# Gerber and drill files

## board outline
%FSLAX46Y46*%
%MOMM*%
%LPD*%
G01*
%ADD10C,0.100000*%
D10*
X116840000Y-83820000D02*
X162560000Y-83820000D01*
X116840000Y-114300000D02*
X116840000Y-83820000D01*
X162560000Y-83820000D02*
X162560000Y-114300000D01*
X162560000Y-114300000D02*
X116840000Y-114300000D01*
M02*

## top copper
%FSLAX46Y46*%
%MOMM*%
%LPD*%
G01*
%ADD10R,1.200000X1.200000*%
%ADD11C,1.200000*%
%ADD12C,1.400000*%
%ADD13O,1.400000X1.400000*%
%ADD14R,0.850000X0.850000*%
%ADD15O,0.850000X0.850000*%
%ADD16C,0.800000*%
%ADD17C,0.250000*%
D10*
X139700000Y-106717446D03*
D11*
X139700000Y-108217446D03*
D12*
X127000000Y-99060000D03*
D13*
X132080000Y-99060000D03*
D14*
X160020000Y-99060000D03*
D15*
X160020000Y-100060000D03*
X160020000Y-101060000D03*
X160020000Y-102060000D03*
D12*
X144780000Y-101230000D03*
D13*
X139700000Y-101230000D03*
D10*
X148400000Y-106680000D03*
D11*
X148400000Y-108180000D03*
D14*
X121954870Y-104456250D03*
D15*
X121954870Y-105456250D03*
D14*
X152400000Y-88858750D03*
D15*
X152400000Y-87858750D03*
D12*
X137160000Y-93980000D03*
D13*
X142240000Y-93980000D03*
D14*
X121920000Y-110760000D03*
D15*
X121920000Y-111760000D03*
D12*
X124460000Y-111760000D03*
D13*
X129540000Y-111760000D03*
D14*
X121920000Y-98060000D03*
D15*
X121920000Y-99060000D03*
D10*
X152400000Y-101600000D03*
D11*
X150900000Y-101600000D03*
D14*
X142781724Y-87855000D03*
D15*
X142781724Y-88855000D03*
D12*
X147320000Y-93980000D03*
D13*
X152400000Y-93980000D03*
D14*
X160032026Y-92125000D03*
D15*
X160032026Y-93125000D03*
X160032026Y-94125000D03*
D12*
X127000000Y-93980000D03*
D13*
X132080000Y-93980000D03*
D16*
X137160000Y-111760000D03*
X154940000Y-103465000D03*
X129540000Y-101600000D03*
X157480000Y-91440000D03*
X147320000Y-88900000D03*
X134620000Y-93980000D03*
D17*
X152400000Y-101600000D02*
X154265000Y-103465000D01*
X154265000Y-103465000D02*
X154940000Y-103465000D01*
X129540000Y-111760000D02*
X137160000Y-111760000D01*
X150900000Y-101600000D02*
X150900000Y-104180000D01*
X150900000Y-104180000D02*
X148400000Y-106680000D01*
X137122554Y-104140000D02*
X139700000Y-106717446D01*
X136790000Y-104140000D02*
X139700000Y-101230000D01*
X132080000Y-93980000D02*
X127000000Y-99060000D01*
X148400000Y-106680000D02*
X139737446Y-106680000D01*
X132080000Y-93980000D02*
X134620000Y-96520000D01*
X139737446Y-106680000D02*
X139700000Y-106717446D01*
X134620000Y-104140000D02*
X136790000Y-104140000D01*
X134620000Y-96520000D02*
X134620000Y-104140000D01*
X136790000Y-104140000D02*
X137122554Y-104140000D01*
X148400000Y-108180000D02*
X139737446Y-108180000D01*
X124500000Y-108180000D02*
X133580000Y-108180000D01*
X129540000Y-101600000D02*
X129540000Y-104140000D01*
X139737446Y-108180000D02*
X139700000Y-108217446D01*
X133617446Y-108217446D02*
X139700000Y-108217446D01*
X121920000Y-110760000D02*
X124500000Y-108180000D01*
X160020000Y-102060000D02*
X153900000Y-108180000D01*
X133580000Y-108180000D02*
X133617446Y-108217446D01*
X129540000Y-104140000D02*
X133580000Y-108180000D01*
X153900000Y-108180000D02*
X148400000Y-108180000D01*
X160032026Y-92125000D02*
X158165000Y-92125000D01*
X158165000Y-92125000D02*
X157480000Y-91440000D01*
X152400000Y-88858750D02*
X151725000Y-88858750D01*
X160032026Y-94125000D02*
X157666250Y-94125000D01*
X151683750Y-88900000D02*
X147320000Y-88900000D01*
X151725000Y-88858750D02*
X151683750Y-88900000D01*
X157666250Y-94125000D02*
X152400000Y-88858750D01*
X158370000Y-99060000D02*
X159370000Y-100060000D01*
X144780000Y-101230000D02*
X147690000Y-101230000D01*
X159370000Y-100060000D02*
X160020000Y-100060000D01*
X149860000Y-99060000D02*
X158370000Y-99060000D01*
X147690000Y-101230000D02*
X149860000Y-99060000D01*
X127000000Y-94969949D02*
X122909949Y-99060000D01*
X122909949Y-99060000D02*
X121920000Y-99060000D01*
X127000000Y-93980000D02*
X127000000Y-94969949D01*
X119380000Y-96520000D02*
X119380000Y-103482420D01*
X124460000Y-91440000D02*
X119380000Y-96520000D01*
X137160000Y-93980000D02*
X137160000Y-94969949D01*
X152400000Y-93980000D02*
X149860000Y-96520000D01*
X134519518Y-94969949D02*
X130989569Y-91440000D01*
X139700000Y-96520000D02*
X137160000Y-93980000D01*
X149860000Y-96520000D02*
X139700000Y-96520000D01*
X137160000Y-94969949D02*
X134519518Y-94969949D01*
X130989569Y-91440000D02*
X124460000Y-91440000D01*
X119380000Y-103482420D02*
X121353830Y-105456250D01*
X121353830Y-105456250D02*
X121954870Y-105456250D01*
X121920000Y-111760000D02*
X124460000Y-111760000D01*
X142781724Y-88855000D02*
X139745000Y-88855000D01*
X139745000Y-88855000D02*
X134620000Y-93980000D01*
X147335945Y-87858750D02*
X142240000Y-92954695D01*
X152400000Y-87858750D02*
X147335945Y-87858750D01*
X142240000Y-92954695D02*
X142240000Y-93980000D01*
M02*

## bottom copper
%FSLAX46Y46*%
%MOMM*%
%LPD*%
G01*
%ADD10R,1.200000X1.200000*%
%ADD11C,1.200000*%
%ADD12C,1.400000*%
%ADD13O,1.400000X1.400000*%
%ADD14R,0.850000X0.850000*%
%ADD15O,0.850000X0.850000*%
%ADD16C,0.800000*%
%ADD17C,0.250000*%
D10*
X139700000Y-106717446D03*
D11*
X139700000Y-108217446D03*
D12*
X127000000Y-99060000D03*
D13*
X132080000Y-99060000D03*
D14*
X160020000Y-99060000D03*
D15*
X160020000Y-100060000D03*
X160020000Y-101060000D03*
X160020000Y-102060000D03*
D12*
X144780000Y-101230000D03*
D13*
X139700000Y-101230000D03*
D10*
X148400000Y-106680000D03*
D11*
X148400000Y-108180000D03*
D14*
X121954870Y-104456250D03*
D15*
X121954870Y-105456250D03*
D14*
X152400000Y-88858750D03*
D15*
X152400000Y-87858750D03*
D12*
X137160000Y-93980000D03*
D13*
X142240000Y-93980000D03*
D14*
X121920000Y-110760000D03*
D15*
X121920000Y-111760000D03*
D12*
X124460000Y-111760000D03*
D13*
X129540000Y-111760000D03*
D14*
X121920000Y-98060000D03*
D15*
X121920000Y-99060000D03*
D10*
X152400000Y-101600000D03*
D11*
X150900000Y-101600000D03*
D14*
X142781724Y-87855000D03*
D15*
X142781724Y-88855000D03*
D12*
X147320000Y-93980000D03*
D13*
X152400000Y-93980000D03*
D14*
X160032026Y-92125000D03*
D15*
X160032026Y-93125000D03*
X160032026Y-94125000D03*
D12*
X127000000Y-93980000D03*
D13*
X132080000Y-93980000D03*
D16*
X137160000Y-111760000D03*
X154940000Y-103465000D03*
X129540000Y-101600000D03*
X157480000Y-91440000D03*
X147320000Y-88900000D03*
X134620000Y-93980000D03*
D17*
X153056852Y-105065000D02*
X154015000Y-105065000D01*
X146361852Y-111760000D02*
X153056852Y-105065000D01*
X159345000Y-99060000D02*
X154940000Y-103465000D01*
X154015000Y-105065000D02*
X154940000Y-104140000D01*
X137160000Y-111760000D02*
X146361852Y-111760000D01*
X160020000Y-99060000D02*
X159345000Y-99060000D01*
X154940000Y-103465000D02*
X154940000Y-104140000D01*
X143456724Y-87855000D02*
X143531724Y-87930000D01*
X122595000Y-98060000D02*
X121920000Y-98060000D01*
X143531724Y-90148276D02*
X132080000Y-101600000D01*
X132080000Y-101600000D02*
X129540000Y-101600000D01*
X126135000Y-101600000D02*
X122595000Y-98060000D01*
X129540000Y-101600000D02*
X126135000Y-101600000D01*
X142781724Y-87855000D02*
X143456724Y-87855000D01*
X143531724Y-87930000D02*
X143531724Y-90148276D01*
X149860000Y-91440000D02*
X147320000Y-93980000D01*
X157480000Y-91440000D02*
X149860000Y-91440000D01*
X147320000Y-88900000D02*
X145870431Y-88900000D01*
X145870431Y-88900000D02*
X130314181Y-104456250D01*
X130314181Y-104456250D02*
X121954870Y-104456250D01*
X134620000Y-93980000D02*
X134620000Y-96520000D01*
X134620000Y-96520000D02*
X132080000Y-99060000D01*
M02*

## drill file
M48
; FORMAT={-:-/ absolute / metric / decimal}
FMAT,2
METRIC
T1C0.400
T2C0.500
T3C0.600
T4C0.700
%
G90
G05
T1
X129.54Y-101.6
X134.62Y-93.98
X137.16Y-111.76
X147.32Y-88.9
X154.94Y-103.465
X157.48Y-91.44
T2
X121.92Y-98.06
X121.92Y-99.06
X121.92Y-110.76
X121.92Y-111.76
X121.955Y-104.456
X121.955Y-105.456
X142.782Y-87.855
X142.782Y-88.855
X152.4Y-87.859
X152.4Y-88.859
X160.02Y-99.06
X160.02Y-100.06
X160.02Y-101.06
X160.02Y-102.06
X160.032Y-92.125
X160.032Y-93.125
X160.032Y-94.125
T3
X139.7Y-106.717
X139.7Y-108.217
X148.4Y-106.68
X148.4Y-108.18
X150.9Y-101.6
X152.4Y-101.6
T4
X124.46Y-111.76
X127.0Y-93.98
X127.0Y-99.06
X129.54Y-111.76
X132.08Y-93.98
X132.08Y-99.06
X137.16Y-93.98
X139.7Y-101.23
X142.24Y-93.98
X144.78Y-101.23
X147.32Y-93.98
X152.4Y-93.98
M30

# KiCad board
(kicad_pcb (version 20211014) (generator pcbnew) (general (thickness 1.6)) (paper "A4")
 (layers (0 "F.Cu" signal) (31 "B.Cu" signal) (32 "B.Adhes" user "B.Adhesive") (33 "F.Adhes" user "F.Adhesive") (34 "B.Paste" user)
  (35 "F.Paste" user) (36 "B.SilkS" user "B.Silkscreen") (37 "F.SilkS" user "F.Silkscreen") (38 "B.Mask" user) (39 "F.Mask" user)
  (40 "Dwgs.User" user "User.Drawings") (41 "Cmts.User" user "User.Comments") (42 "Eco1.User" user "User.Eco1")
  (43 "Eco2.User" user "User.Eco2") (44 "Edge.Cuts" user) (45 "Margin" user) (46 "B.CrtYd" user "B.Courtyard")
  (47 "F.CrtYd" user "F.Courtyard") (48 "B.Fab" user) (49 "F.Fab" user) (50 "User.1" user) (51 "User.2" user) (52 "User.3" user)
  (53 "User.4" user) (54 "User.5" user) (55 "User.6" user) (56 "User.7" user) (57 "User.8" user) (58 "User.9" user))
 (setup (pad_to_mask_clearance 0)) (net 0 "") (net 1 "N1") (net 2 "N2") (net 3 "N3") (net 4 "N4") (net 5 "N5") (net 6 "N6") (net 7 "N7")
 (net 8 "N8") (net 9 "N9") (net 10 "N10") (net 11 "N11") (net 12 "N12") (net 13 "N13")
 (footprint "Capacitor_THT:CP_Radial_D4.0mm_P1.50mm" (layer "F.Cu") (at 139.7 106.717446 -90)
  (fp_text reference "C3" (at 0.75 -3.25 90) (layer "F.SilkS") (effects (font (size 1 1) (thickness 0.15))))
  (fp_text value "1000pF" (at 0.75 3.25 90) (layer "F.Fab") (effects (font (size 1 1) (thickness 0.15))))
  (pad "1" thru_hole rect (at 0 0 270) (size 1.2 1.2) (drill 0.6) (layers *.Cu *.Mask) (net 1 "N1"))
  (pad "2" thru_hole circle (at 1.5 0 270) (size 1.2 1.2) (drill 0.6) (layers *.Cu *.Mask) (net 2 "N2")))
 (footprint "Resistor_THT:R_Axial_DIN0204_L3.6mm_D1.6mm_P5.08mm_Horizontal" (layer "F.Cu") (at 127 99.06)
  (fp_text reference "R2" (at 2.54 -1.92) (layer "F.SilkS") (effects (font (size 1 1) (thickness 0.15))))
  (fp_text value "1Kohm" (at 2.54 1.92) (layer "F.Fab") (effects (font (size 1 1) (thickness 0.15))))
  (pad "1" thru_hole circle (at 0 0) (size 1.4 1.4) (drill 0.7) (layers *.Cu *.Mask) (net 1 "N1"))
  (pad "2" thru_hole oval (at 5.08 0) (size 1.4 1.4) (drill 0.7) (layers *.Cu *.Mask) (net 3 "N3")))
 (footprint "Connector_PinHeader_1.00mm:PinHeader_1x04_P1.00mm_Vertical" (layer "F.Cu") (at 160.02 99.06)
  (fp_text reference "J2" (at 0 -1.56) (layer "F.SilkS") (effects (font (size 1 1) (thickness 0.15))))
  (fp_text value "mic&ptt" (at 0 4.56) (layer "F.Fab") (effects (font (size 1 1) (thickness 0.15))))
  (pad "1" thru_hole rect (at 0 0) (size 0.85 0.85) (drill 0.5) (layers *.Cu *.Mask) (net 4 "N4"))
  (pad "2" thru_hole oval (at 0 1) (size 0.85 0.85) (drill 0.5) (layers *.Cu *.Mask) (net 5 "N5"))
  (pad "3" thru_hole oval (at 0 2) (size 0.85 0.85) (drill 0.5) (layers *.Cu *.Mask) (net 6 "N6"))
  (pad "4" thru_hole oval (at 0 3) (size 0.85 0.85) (drill 0.5) (layers *.Cu *.Mask) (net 2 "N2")))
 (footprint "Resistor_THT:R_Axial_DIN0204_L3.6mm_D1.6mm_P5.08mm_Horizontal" (layer "F.Cu") (at 144.78 101.23 180)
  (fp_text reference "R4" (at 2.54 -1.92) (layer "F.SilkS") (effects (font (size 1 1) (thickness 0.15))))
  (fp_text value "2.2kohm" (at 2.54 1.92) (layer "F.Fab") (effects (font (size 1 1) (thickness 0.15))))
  (pad "1" thru_hole circle (at 0 0 180) (size 1.4 1.4) (drill 0.7) (layers *.Cu *.Mask) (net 5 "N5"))
  (pad "2" thru_hole oval (at 5.08 0 180) (size 1.4 1.4) (drill 0.7) (layers *.Cu *.Mask) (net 1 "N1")))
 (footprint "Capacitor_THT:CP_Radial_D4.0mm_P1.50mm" (layer "F.Cu") (at 148.4 106.68 -90)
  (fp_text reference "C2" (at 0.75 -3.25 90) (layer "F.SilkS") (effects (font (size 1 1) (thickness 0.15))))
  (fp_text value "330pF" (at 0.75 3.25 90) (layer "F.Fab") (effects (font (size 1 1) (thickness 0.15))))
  (pad "1" thru_hole rect (at 0 0 270) (size 1.2 1.2) (drill 0.6) (layers *.Cu *.Mask) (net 1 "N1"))
  (pad "2" thru_hole circle (at 1.5 0 270) (size 1.2 1.2) (drill 0.6) (layers *.Cu *.Mask) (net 2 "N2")))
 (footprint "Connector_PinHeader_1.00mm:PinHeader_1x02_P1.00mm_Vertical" (layer "F.Cu") (at 121.95487 104.45625)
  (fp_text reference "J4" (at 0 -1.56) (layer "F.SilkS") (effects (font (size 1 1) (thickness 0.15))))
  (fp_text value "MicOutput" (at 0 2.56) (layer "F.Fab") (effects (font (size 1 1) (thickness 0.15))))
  (pad "1" thru_hole rect (at 0 0) (size 0.85 0.85) (drill 0.5) (layers *.Cu *.Mask) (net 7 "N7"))
  (pad "2" thru_hole oval (at 0 1) (size 0.85 0.85) (drill 0.5) (layers *.Cu *.Mask) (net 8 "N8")))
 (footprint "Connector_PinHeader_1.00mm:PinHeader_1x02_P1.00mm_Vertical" (layer "F.Cu") (at 152.4 88.85875 180)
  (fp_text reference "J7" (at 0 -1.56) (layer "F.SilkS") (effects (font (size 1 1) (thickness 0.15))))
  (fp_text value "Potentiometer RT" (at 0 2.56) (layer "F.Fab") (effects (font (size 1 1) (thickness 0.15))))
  (pad "1" thru_hole rect (at 0 0 180) (size 0.85 0.85) (drill 0.5) (layers *.Cu *.Mask) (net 7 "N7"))
  (pad "2" thru_hole oval (at 0 1 180) (size 0.85 0.85) (drill 0.5) (layers *.Cu *.Mask) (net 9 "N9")))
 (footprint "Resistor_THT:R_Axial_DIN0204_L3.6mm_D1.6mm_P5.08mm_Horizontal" (layer "F.Cu") (at 137.16 93.98)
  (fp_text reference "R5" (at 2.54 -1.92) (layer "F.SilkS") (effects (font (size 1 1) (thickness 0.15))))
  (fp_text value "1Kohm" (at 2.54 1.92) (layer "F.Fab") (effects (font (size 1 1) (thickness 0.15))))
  (pad "1" thru_hole circle (at 0 0) (size 1.4 1.4) (drill 0.7) (layers *.Cu *.Mask) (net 8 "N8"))
  (pad "2" thru_hole oval (at 5.08 0) (size 1.4 1.4) (drill 0.7) (layers *.Cu *.Mask) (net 9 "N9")))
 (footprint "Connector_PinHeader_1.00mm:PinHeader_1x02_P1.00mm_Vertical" (layer "F.Cu") (at 121.92 110.76)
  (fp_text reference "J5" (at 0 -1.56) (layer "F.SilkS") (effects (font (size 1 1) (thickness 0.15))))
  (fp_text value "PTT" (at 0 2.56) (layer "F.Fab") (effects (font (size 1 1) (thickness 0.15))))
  (pad "1" thru_hole rect (at 0 0) (size 0.85 0.85) (drill 0.5) (layers *.Cu *.Mask) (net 2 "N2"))
  (pad "2" thru_hole oval (at 0 1) (size 0.85 0.85) (drill 0.5) (layers *.Cu *.Mask) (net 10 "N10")))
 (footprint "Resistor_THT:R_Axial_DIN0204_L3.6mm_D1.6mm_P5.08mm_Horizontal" (layer "F.Cu") (at 124.46 111.76)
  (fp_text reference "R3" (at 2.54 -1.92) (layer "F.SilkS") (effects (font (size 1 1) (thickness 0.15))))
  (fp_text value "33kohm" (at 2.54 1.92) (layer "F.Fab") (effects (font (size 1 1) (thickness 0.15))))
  (pad "1" thru_hole circle (at 0 0) (size 1.4 1.4) (drill 0.7) (layers *.Cu *.Mask) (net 10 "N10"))
  (pad "2" thru_hole oval (at 5.08 0) (size 1.4 1.4) (drill 0.7) (layers *.Cu *.Mask) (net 4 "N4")))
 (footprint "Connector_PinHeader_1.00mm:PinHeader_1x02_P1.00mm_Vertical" (layer "F.Cu") (at 121.92 98.06)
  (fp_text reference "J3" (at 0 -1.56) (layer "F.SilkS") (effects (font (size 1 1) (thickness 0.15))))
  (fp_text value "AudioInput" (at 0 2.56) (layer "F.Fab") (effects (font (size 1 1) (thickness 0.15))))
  (pad "1" thru_hole rect (at 0 0) (size 0.85 0.85) (drill 0.5) (layers *.Cu *.Mask) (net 2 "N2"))
  (pad "2" thru_hole oval (at 0 1) (size 0.85 0.85) (drill 0.5) (layers *.Cu *.Mask) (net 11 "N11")))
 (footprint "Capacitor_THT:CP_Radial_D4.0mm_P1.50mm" (layer "F.Cu") (at 152.4 101.6 180)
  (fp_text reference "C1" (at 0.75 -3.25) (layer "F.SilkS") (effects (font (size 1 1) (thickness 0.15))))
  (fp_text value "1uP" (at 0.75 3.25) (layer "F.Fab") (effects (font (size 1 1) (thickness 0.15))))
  (pad "1" thru_hole rect (at 0 0 180) (size 1.2 1.2) (drill 0.6) (layers *.Cu *.Mask) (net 4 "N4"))
  (pad "2" thru_hole circle (at 1.5 0 180) (size 1.2 1.2) (drill 0.6) (layers *.Cu *.Mask) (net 1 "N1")))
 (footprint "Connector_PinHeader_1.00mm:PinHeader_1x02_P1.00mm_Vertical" (layer "F.Cu") (at 142.781724 87.855)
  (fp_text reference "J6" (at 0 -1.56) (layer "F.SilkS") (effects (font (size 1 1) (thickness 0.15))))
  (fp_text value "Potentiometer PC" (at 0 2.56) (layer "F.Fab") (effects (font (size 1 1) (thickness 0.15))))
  (pad "1" thru_hole rect (at 0 0) (size 0.85 0.85) (drill 0.5) (layers *.Cu *.Mask) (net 2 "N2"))
  (pad "2" thru_hole oval (at 0 1) (size 0.85 0.85) (drill 0.5) (layers *.Cu *.Mask) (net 3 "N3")))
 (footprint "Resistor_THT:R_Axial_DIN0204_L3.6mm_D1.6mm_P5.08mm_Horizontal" (layer "F.Cu") (at 147.32 93.98)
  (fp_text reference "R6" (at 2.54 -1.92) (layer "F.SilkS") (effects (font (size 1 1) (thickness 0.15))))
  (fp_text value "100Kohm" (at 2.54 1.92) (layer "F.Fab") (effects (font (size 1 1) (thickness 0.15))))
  (pad "1" thru_hole circle (at 0 0) (size 1.4 1.4) (drill 0.7) (layers *.Cu *.Mask) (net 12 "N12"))
  (pad "2" thru_hole oval (at 5.08 0) (size 1.4 1.4) (drill 0.7) (layers *.Cu *.Mask) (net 8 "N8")))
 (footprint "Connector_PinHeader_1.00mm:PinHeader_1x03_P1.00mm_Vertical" (layer "F.Cu") (at 160.032026 92.125)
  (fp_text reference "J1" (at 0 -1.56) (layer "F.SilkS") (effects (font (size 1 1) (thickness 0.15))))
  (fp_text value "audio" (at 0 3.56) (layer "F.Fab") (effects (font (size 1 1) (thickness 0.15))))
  (pad "1" thru_hole rect (at 0 0) (size 0.85 0.85) (drill 0.5) (layers *.Cu *.Mask) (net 12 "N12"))
  (pad "2" thru_hole oval (at 0 1) (size 0.85 0.85) (drill 0.5) (layers *.Cu *.Mask) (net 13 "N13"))
  (pad "3" thru_hole oval (at 0 2) (size 0.85 0.85) (drill 0.5) (layers *.Cu *.Mask) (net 7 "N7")))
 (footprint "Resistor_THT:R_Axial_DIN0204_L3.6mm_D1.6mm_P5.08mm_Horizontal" (layer "F.Cu") (at 127 93.98)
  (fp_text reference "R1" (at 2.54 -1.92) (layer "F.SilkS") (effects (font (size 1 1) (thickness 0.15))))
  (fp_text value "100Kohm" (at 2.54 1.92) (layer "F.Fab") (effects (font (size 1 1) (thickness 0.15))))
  (pad "1" thru_hole circle (at 0 0) (size 1.4 1.4) (drill 0.7) (layers *.Cu *.Mask) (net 11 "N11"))
  (pad "2" thru_hole oval (at 5.08 0) (size 1.4 1.4) (drill 0.7) (layers *.Cu *.Mask) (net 1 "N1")))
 (gr_line (start 116.84 83.82) (end 162.56 83.82) (layer "Edge.Cuts") (width 0.1))
 (gr_line (start 116.84 114.3) (end 116.84 83.82) (layer "Edge.Cuts") (width 0.1))
 (gr_line (start 162.56 83.82) (end 162.56 114.3) (layer "Edge.Cuts") (width 0.1))
 (gr_line (start 162.56 114.3) (end 116.84 114.3) (layer "Edge.Cuts") (width 0.1))
 (segment (start 152.4 101.6) (end 154.265 103.465) (width 0.25) (layer "F.Cu") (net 4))
 (segment (start 154.265 103.465) (end 154.94 103.465) (width 0.25) (layer "F.Cu") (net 4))
 (segment (start 129.54 111.76) (end 137.16 111.76) (width 0.25) (layer "F.Cu") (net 4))
 (via (at 137.16 111.76) (size 0.8) (drill 0.4) (layers "F.Cu" "B.Cu") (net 4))
 (via (at 154.94 103.465) (size 0.8) (drill 0.4) (layers "F.Cu" "B.Cu") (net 4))
 (segment (start 153.056852 105.065) (end 154.015 105.065) (width 0.25) (layer "B.Cu") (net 4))
 (segment (start 146.361852 111.76) (end 153.056852 105.065) (width 0.25) (layer "B.Cu") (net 4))
 (segment (start 159.345 99.06) (end 154.94 103.465) (width 0.25) (layer "B.Cu") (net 4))
 (segment (start 154.015 105.065) (end 154.94 104.14) (width 0.25) (layer "B.Cu") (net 4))
 (segment (start 137.16 111.76) (end 146.361852 111.76) (width 0.25) (layer "B.Cu") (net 4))
 (segment (start 160.02 99.06) (end 159.345 99.06) (width 0.25) (layer "B.Cu") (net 4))
 (segment (start 154.94 103.465) (end 154.94 104.14) (width 0.25) (layer "B.Cu") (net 4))
 (segment (start 150.9 101.6) (end 150.9 104.18) (width 0.25) (layer "F.Cu") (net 1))
 (segment (start 150.9 104.18) (end 148.4 106.68) (width 0.25) (layer "F.Cu") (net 1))
 (segment (start 137.122554 104.14) (end 139.7 106.717446) (width 0.25) (layer "F.Cu") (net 1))
 (segment (start 136.79 104.14) (end 139.7 101.23) (width 0.25) (layer "F.Cu") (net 1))
 (segment (start 132.08 93.98) (end 127 99.06) (width 0.25) (layer "F.Cu") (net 1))
 (segment (start 148.4 106.68) (end 139.737446 106.68) (width 0.25) (layer "F.Cu") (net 1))
 (segment (start 132.08 93.98) (end 134.62 96.52) (width 0.25) (layer "F.Cu") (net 1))
 (segment (start 139.737446 106.68) (end 139.7 106.717446) (width 0.25) (layer "F.Cu") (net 1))
 (segment (start 134.62 104.14) (end 136.79 104.14) (width 0.25) (layer "F.Cu") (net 1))
 (segment (start 134.62 96.52) (end 134.62 104.14) (width 0.25) (layer "F.Cu") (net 1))
 (segment (start 136.79 104.14) (end 137.122554 104.14) (width 0.25) (layer "F.Cu") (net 1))
 (segment (start 148.4 108.18) (end 139.737446 108.18) (width 0.25) (layer "F.Cu") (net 2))
 (segment (start 124.5 108.18) (end 133.58 108.18) (width 0.25) (layer "F.Cu") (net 2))
 (segment (start 129.54 101.6) (end 129.54 104.14) (width 0.25) (layer "F.Cu") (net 2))
 (segment (start 139.737446 108.18) (end 139.7 108.217446) (width 0.25) (layer "F.Cu") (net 2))
 (segment (start 133.617446 108.217446) (end 139.7 108.217446) (width 0.25) (layer "F.Cu") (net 2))
 (segment (start 121.92 110.76) (end 124.5 108.18) (width 0.25) (layer "F.Cu") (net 2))
 (segment (start 160.02 102.06) (end 153.9 108.18) (width 0.25) (layer "F.Cu") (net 2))
 (segment (start 133.58 108.18) (end 133.617446 108.217446) (width 0.25) (layer "F.Cu") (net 2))
 (segment (start 129.54 104.14) (end 133.58 108.18) (width 0.25) (layer "F.Cu") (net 2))
 (segment (start 153.9 108.18) (end 148.4 108.18) (width 0.25) (layer "F.Cu") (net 2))
 (via (at 129.54 101.6) (size 0.8) (drill 0.4) (layers "F.Cu" "B.Cu") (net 2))
 (segment (start 143.456724 87.855) (end 143.531724 87.93) (width 0.25) (layer "B.Cu") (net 2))
 (segment (start 122.595 98.06) (end 121.92 98.06) (width 0.25) (layer "B.Cu") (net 2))
 (segment (start 143.531724 90.148276) (end 132.08 101.6) (width 0.25) (layer "B.Cu") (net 2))
 (segment (start 132.08 101.6) (end 129.54 101.6) (width 0.25) (layer "B.Cu") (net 2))
 (segment (start 126.135 101.6) (end 122.595 98.06) (width 0.25) (layer "B.Cu") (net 2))
 (segment (start 129.54 101.6) (end 126.135 101.6) (width 0.25) (layer "B.Cu") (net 2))
 (segment (start 142.781724 87.855) (end 143.456724 87.855) (width 0.25) (layer "B.Cu") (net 2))
 (segment (start 143.531724 87.93) (end 143.531724 90.148276) (width 0.25) (layer "B.Cu") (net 2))
 (segment (start 160.032026 92.125) (end 158.165 92.125) (width 0.25) (layer "F.Cu") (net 12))
 (segment (start 158.165 92.125) (end 157.48 91.44) (width 0.25) (layer "F.Cu") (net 12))
 (via (at 157.48 91.44) (size 0.8) (drill 0.4) (layers "F.Cu" "B.Cu") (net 12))
 (segment (start 149.86 91.44) (end 147.32 93.98) (width 0.25) (layer "B.Cu") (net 12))
 (segment (start 157.48 91.44) (end 149.86 91.44) (width 0.25) (layer "B.Cu") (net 12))
 (segment (start 152.4 88.85875) (end 151.725 88.85875) (width 0.25) (layer "F.Cu") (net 7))
 (segment (start 160.032026 94.125) (end 157.66625 94.125) (width 0.25) (layer "F.Cu") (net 7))
 (segment (start 151.68375 88.9) (end 147.32 88.9) (width 0.25) (layer "F.Cu") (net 7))
 (segment (start 151.725 88.85875) (end 151.68375 88.9) (width 0.25) (layer "F.Cu") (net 7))
 (segment (start 157.66625 94.125) (end 152.4 88.85875) (width 0.25) (layer "F.Cu") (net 7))
 (via (at 147.32 88.9) (size 0.8) (drill 0.4) (layers "F.Cu" "B.Cu") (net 7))
 (segment (start 147.32 88.9) (end 145.870431 88.9) (width 0.25) (layer "B.Cu") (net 7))
 (segment (start 145.870431 88.9) (end 130.314181 104.45625) (width 0.25) (layer "B.Cu") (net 7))
 (segment (start 130.314181 104.45625) (end 121.95487 104.45625) (width 0.25) (layer "B.Cu") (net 7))
 (segment (start 158.37 99.06) (end 159.37 100.06) (width 0.25) (layer "F.Cu") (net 5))
 (segment (start 144.78 101.23) (end 147.69 101.23) (width 0.25) (layer "F.Cu") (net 5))
 (segment (start 159.37 100.06) (end 160.02 100.06) (width 0.25) (layer "F.Cu") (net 5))
 (segment (start 149.86 99.06) (end 158.37 99.06) (width 0.25) (layer "F.Cu") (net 5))
 (segment (start 147.69 101.23) (end 149.86 99.06) (width 0.25) (layer "F.Cu") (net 5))
 (segment (start 127 94.969949) (end 122.909949 99.06) (width 0.25) (layer "F.Cu") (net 11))
 (segment (start 122.909949 99.06) (end 121.92 99.06) (width 0.25) (layer "F.Cu") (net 11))
 (segment (start 127 93.98) (end 127 94.969949) (width 0.25) (layer "F.Cu") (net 11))
 (segment (start 119.38 96.52) (end 119.38 103.48242) (width 0.25) (layer "F.Cu") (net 8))
 (segment (start 124.46 91.44) (end 119.38 96.52) (width 0.25) (layer "F.Cu") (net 8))
 (segment (start 137.16 93.98) (end 137.16 94.969949) (width 0.25) (layer "F.Cu") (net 8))
 (segment (start 152.4 93.98) (end 149.86 96.52) (width 0.25) (layer "F.Cu") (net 8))
 (segment (start 134.519518 94.969949) (end 130.989569 91.44) (width 0.25) (layer "F.Cu") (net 8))
 (segment (start 139.7 96.52) (end 137.16 93.98) (width 0.25) (layer "F.Cu") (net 8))
 (segment (start 149.86 96.52) (end 139.7 96.52) (width 0.25) (layer "F.Cu") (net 8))
 (segment (start 137.16 94.969949) (end 134.519518 94.969949) (width 0.25) (layer "F.Cu") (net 8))
 (segment (start 130.989569 91.44) (end 124.46 91.44) (width 0.25) (layer "F.Cu") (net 8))
 (segment (start 119.38 103.48242) (end 121.35383 105.45625) (width 0.25) (layer "F.Cu") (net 8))
 (segment (start 121.35383 105.45625) (end 121.95487 105.45625) (width 0.25) (layer "F.Cu") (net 8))
 (segment (start 121.92 111.76) (end 124.46 111.76) (width 0.25) (layer "F.Cu") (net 10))
 (segment (start 142.781724 88.855) (end 139.745 88.855) (width 0.25) (layer "F.Cu") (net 3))
 (segment (start 139.745 88.855) (end 134.62 93.98) (width 0.25) (layer "F.Cu") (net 3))
 (via (at 134.62 93.98) (size 0.8) (drill 0.4) (layers "F.Cu" "B.Cu") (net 3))
 (segment (start 134.62 93.98) (end 134.62 96.52) (width 0.25) (layer "B.Cu") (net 3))
 (segment (start 134.62 96.52) (end 132.08 99.06) (width 0.25) (layer "B.Cu") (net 3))
 (segment (start 147.335945 87.85875) (end 142.24 92.954695) (width 0.25) (layer "F.Cu") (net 9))
 (segment (start 152.4 87.85875) (end 147.335945 87.85875) (width 0.25) (layer "F.Cu") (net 9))
 (segment (start 142.24 92.954695) (end 142.24 93.98) (width 0.25) (layer "F.Cu") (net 9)))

